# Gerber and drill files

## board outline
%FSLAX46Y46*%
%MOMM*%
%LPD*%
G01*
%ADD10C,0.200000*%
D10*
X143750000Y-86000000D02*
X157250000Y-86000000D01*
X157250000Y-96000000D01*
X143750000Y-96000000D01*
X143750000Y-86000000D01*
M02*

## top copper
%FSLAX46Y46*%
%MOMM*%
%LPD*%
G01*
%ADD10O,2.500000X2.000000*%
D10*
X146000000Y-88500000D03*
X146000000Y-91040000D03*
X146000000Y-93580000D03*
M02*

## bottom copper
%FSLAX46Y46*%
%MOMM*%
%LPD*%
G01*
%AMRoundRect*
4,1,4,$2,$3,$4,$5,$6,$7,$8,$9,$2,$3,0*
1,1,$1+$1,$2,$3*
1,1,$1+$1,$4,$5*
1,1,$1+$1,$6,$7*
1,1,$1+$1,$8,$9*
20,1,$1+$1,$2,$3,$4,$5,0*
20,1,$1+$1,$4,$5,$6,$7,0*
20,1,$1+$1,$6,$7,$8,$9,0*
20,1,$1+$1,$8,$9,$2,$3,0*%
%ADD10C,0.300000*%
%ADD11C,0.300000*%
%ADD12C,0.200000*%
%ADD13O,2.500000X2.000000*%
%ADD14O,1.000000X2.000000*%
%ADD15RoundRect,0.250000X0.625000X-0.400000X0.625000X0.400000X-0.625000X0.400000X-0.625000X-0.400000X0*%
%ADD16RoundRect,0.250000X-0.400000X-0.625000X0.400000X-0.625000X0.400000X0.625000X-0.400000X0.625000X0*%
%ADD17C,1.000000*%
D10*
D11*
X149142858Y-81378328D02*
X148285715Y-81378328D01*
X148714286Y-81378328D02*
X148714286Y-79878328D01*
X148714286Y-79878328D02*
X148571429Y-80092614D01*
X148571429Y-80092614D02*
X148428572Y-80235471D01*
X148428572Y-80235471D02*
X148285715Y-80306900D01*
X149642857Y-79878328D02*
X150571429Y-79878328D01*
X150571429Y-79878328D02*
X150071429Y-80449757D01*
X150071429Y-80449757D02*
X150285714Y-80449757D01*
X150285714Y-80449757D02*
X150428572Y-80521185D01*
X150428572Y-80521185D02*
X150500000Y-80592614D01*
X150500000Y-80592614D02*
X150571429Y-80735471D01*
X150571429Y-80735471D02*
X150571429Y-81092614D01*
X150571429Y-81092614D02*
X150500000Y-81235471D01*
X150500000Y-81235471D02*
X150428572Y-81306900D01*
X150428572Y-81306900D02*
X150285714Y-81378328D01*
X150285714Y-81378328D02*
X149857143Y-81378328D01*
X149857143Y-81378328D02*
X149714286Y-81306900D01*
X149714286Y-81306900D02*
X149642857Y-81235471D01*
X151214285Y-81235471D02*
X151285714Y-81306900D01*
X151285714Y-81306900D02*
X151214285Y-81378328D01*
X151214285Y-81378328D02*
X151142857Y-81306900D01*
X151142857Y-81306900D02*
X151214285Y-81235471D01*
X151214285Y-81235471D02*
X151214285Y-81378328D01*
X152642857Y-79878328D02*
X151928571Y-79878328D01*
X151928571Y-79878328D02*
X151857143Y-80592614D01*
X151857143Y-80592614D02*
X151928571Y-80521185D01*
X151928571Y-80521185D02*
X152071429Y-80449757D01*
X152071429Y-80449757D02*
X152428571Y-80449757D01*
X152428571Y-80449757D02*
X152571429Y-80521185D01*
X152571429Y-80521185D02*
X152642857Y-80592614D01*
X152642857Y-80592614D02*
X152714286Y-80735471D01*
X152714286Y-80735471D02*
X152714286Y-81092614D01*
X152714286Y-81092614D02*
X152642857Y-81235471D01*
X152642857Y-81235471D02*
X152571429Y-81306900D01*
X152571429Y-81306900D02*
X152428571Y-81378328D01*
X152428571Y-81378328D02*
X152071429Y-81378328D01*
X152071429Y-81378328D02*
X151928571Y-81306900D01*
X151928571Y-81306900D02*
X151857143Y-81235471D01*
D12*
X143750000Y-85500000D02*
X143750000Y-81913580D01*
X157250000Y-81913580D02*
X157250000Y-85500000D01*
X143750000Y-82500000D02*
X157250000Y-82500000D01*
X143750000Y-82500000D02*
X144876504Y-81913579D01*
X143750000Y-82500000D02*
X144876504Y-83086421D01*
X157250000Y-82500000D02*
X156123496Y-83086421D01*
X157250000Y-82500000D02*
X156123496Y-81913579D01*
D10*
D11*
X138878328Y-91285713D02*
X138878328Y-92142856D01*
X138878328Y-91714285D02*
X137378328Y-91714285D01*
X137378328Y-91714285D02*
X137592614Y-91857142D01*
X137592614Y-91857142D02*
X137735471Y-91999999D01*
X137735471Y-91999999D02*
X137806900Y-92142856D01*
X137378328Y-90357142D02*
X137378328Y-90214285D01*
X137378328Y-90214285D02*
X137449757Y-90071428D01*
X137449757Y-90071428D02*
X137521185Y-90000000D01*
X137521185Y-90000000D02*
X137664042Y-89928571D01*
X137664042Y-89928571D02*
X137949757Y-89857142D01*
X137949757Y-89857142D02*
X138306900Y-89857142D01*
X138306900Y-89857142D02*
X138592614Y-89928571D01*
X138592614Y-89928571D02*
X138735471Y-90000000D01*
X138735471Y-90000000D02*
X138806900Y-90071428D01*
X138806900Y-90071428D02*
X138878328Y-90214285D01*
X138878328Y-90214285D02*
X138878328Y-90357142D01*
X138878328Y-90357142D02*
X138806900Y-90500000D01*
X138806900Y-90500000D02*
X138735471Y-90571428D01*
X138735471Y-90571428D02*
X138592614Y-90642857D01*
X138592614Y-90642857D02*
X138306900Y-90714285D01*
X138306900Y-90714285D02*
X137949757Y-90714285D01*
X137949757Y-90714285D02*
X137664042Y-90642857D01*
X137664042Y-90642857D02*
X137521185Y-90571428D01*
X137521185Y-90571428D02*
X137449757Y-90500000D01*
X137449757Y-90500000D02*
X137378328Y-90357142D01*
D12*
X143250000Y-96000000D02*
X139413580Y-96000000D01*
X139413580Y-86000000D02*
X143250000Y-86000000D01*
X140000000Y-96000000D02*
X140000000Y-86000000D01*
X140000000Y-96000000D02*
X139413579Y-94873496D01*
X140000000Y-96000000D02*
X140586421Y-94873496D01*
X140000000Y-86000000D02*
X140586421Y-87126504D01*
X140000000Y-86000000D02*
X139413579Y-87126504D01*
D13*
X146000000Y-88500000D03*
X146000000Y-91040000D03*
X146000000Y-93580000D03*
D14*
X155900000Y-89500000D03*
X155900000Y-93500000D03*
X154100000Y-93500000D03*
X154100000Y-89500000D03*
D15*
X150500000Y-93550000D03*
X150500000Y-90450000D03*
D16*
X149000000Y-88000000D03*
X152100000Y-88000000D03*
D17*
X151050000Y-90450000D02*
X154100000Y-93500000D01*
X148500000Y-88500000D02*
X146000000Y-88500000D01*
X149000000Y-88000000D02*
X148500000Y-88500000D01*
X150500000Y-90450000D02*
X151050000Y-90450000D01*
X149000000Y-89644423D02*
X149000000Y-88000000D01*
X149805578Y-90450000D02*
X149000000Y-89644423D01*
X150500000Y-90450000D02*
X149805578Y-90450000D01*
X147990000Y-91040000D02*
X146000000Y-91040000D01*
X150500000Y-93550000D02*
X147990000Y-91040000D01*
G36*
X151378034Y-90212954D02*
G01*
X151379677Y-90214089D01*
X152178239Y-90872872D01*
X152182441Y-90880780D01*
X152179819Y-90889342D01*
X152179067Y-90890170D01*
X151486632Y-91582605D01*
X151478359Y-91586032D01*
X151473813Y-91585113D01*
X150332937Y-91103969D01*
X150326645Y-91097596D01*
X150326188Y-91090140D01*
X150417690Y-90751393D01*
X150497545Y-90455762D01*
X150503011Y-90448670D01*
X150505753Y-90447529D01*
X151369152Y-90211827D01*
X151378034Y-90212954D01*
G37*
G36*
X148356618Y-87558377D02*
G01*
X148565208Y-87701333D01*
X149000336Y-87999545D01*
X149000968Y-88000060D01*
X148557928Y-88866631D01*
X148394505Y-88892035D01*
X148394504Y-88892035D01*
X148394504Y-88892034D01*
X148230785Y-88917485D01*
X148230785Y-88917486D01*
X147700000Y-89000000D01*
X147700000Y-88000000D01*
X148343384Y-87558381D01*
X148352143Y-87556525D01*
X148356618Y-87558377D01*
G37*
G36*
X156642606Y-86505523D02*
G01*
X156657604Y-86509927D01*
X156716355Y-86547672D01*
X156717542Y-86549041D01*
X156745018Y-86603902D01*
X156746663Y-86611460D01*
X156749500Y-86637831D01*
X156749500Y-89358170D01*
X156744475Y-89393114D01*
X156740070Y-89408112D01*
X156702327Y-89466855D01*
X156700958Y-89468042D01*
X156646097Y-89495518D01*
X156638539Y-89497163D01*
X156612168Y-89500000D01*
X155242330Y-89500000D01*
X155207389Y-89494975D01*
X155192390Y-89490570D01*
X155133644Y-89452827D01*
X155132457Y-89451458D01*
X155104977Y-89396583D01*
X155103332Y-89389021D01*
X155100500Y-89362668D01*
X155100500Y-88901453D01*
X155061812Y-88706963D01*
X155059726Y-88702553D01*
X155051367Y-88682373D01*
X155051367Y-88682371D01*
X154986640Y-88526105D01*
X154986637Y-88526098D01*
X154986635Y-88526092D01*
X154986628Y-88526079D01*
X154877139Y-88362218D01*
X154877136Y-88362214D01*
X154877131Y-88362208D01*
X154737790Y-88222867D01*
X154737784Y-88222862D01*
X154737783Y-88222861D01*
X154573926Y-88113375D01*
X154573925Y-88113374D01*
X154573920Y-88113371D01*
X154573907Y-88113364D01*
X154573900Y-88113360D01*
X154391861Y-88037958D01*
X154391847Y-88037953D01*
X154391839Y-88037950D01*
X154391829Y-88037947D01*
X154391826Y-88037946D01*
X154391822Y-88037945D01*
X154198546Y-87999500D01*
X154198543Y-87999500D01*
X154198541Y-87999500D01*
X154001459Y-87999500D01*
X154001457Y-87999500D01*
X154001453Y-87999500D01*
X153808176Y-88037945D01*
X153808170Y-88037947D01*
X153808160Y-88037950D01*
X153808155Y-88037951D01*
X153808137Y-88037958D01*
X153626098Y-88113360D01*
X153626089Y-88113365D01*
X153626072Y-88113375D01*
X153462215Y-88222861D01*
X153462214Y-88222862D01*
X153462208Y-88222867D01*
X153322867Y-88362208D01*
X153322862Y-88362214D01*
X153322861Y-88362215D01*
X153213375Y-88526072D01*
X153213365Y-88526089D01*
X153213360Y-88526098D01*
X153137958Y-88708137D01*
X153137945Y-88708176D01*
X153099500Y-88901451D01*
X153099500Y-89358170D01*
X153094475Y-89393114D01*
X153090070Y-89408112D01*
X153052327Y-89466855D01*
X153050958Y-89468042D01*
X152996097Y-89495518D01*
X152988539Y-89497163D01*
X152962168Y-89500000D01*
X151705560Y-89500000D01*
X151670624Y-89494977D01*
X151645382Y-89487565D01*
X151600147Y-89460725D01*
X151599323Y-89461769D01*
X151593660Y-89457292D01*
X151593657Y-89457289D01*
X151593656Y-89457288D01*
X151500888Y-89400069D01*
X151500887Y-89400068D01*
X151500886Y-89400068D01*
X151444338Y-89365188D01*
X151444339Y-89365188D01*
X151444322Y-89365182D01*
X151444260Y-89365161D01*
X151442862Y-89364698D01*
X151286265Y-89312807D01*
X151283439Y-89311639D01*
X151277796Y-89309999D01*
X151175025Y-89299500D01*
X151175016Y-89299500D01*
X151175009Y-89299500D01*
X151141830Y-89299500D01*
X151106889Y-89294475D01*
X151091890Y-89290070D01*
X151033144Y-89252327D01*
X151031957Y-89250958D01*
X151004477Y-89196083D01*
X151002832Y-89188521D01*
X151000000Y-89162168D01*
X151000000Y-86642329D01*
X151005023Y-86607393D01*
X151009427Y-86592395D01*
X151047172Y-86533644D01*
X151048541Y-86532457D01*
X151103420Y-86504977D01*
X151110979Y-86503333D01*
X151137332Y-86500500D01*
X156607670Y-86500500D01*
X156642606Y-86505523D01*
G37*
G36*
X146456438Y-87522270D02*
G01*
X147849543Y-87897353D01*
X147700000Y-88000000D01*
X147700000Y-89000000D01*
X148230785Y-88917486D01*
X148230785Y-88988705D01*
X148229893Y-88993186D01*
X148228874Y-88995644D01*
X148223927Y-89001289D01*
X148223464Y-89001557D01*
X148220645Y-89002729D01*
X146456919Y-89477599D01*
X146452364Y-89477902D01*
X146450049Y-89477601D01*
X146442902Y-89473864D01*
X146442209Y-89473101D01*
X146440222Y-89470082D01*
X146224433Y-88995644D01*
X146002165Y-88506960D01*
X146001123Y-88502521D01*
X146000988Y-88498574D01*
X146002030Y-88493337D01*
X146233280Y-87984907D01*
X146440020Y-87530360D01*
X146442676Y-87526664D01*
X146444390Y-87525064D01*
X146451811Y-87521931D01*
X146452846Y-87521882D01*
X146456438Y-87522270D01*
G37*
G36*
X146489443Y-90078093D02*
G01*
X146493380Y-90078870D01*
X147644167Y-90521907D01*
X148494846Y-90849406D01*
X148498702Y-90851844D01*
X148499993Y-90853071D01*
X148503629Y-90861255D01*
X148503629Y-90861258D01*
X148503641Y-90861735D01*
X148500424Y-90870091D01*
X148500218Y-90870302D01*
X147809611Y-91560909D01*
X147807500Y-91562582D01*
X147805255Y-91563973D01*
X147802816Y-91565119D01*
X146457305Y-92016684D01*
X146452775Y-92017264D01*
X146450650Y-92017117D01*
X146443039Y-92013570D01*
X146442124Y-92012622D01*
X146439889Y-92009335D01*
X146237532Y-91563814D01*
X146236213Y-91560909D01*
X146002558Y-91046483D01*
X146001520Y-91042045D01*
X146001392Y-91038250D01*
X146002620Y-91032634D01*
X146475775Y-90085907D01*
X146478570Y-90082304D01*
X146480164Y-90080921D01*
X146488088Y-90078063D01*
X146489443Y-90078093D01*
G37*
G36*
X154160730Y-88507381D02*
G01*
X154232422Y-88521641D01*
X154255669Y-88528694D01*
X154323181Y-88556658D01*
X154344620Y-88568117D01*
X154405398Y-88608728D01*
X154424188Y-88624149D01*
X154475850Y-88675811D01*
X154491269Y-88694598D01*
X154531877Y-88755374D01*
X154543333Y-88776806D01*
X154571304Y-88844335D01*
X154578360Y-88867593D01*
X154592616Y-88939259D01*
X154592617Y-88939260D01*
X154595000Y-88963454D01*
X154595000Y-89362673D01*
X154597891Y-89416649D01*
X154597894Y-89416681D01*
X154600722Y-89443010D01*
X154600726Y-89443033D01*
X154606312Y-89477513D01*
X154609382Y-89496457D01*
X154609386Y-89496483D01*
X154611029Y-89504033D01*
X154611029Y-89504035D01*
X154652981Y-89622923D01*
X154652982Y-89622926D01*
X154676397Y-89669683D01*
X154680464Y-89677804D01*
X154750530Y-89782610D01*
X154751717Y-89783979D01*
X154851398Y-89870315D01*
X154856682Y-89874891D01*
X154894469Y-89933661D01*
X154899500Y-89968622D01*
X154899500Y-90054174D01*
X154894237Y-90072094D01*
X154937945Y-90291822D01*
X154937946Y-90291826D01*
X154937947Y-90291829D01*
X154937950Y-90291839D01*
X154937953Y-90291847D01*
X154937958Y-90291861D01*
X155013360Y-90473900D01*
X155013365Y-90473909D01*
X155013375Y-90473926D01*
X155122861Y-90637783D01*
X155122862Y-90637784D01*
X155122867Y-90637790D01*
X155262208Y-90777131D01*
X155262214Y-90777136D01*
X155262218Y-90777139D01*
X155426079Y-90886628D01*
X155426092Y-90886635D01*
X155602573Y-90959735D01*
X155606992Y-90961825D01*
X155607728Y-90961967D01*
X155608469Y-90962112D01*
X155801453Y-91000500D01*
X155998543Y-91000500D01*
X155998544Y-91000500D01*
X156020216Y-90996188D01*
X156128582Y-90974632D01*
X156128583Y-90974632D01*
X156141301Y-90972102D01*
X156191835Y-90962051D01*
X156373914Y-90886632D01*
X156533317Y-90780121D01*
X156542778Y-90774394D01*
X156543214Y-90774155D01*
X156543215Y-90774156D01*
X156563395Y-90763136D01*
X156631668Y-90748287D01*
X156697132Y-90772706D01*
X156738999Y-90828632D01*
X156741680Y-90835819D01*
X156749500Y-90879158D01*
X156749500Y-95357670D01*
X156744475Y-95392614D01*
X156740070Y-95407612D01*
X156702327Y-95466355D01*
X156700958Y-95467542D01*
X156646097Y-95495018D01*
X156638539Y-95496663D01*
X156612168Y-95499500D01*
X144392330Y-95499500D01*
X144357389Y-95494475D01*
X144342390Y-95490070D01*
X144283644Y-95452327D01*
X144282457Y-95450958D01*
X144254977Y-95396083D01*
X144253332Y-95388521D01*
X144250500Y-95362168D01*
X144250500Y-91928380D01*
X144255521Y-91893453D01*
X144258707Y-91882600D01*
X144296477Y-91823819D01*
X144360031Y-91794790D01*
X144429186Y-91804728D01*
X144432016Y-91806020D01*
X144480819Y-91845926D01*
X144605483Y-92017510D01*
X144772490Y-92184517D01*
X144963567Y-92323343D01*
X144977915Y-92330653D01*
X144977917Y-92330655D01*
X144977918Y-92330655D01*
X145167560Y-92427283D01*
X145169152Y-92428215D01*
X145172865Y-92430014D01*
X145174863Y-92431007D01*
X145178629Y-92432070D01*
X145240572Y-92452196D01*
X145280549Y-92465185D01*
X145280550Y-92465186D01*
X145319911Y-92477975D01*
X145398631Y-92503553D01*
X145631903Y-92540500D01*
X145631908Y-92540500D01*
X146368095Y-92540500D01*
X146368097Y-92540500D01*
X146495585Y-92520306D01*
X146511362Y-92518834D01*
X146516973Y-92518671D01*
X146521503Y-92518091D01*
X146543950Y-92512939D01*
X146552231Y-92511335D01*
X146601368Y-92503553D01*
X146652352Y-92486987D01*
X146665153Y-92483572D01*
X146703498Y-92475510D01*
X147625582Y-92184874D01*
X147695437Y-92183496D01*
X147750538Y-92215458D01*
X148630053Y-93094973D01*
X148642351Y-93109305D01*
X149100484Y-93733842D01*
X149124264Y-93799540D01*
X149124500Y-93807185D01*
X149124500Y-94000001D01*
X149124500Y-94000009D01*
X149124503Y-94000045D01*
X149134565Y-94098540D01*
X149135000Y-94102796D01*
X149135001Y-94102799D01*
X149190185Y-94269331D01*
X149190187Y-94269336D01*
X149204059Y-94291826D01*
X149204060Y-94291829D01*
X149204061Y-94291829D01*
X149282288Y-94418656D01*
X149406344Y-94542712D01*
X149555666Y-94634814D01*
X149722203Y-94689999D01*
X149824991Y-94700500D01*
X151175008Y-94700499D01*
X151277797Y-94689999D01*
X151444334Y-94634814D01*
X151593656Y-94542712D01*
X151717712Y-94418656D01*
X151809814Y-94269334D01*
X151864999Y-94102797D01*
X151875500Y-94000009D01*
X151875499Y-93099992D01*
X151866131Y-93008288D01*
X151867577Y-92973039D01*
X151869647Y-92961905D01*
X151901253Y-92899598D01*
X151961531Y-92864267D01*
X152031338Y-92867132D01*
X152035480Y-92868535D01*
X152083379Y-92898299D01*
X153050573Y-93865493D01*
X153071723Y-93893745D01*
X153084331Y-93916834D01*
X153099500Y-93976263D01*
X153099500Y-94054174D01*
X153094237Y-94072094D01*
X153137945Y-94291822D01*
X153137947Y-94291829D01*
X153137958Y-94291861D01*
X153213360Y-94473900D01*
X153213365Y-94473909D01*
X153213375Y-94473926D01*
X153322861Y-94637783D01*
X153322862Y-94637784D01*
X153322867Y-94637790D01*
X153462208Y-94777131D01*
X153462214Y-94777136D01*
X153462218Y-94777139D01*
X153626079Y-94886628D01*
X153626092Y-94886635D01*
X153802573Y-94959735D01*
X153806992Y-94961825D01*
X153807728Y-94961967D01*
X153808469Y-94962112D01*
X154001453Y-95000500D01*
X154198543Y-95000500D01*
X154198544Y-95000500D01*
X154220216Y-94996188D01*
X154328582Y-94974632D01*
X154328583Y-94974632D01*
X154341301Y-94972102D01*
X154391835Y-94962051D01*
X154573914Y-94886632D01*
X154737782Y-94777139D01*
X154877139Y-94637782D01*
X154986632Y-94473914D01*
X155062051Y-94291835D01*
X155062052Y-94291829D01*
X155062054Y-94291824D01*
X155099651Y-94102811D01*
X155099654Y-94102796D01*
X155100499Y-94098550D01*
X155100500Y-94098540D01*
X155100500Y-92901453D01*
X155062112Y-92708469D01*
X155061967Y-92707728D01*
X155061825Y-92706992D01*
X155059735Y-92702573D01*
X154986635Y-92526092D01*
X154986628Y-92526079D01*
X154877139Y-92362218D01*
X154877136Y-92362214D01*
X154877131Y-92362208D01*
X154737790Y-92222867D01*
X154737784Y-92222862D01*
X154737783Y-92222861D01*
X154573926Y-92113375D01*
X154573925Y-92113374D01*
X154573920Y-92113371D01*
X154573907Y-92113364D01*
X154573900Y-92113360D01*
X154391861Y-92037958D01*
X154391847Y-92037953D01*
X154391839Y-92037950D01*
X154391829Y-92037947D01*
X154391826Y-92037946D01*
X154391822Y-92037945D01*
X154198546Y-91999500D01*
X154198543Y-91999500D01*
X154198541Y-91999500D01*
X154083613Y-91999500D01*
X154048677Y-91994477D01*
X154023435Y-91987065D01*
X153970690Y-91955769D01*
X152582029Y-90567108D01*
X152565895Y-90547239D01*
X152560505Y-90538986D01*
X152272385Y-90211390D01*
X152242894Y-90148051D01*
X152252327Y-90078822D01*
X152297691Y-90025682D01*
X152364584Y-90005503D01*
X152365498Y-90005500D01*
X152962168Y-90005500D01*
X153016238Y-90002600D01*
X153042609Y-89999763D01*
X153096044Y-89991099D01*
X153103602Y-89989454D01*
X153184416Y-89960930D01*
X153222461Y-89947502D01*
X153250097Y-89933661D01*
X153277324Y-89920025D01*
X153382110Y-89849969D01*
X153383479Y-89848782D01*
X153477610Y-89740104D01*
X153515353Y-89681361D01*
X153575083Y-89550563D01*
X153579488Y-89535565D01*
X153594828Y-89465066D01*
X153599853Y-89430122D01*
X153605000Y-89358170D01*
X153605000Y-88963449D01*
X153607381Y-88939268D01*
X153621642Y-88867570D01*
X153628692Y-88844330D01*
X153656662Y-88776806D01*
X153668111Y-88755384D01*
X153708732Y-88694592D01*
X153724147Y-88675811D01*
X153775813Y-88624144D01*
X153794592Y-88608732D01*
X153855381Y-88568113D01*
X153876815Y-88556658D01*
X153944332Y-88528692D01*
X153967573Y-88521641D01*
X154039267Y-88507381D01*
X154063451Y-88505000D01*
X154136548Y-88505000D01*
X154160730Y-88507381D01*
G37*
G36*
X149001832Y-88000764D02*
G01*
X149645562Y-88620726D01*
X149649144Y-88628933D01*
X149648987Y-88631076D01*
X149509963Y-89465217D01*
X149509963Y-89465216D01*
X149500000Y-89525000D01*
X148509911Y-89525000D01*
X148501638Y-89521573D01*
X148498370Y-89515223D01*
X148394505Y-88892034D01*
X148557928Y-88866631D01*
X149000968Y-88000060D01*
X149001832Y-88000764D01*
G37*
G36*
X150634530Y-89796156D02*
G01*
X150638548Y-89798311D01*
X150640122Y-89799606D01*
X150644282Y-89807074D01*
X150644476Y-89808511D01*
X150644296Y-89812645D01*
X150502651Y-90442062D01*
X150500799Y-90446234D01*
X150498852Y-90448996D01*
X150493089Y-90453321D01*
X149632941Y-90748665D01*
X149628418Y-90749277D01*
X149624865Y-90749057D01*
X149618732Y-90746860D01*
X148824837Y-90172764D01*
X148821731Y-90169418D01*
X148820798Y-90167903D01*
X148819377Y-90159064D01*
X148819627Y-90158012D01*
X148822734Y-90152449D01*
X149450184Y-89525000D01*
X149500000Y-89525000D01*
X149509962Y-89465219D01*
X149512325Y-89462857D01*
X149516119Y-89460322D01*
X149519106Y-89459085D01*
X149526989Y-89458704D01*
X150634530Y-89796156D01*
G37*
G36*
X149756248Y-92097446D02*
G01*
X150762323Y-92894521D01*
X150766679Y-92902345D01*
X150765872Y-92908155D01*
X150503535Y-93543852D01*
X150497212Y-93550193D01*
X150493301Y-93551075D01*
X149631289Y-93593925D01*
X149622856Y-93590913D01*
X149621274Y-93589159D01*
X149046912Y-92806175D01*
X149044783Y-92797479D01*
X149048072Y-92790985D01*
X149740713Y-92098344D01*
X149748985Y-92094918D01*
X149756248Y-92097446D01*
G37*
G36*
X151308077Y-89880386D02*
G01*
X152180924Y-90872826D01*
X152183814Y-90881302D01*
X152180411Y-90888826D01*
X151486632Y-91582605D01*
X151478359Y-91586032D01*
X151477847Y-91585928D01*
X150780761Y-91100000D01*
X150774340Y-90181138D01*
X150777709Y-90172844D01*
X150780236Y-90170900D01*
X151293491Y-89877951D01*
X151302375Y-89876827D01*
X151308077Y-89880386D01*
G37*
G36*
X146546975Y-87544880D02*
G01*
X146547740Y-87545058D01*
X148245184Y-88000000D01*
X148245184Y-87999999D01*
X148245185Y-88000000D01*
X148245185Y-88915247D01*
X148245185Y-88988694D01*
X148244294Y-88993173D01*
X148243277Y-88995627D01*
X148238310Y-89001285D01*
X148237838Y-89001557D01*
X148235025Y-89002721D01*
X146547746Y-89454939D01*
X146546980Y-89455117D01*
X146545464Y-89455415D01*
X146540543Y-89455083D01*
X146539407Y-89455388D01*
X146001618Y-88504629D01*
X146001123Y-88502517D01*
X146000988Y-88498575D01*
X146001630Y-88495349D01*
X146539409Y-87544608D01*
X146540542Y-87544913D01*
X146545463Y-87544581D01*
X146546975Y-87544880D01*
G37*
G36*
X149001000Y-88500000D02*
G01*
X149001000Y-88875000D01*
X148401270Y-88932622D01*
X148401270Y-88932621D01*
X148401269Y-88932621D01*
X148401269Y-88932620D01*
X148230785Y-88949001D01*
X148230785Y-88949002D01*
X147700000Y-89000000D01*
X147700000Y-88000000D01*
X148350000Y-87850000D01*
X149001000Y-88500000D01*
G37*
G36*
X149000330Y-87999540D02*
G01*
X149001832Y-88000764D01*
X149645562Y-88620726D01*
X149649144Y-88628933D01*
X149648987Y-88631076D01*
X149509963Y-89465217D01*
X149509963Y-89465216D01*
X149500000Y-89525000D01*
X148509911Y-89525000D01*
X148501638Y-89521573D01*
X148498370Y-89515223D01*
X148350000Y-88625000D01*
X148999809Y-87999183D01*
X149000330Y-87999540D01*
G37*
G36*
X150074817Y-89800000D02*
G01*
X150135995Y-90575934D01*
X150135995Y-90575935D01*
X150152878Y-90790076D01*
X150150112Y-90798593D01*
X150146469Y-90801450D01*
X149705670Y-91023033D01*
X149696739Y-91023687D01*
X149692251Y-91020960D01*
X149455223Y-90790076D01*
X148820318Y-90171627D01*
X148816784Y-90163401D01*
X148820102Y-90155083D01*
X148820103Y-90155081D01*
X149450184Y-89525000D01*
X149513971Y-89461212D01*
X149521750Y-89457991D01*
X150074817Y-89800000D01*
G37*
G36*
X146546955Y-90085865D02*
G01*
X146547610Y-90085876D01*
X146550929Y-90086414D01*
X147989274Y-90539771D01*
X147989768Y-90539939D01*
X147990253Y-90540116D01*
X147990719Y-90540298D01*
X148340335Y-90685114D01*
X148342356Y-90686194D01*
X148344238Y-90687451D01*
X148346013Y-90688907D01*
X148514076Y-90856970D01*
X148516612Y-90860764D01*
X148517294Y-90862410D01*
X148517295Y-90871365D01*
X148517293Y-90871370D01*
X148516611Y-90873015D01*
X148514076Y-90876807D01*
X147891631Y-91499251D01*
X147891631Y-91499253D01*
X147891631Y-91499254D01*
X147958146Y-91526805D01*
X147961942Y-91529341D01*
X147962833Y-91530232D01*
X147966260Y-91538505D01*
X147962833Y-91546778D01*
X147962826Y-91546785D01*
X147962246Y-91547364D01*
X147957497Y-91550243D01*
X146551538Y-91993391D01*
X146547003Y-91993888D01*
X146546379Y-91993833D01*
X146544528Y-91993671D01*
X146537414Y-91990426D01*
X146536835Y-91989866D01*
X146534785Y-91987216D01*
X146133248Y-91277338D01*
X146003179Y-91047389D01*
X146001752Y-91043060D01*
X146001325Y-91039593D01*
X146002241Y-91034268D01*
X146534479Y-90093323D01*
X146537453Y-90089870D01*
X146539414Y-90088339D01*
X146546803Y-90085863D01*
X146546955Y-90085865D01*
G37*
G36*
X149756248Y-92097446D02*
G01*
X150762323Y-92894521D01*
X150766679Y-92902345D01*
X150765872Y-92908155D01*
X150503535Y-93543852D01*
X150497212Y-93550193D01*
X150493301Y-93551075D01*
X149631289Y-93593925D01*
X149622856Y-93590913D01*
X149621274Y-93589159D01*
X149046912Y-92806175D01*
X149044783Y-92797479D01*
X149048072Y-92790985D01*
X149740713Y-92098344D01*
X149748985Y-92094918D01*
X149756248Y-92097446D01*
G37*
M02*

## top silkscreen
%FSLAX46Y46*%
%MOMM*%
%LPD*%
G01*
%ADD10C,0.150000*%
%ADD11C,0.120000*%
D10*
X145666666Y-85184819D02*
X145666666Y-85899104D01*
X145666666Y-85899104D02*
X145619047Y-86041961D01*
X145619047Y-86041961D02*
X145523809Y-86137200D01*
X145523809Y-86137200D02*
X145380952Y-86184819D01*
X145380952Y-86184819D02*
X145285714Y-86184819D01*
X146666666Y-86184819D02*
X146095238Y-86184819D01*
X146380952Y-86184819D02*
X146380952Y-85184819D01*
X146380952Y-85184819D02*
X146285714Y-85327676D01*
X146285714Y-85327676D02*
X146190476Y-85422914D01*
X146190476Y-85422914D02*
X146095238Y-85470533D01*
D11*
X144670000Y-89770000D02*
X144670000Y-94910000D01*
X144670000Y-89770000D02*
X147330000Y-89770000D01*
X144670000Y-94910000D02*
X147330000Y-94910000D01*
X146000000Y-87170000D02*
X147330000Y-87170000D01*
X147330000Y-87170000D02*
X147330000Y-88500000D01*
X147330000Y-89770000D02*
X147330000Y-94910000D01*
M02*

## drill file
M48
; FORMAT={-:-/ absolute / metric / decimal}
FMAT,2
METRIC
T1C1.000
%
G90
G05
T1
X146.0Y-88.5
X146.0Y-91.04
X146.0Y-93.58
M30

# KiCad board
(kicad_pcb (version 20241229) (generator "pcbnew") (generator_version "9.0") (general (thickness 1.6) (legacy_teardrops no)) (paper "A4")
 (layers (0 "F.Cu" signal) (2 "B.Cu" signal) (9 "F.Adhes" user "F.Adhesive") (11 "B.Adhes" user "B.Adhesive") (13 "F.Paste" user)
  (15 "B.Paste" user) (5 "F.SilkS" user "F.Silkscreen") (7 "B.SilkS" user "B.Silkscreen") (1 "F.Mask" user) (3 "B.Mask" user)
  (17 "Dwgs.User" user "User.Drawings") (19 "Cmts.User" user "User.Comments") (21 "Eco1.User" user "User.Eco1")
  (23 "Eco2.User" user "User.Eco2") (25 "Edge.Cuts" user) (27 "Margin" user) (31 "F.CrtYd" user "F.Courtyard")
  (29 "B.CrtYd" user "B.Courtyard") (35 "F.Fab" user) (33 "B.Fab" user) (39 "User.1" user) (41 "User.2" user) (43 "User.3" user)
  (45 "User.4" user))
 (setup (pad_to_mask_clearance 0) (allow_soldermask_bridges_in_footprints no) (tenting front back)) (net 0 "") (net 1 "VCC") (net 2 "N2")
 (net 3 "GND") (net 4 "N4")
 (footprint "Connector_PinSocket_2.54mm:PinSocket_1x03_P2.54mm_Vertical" (layer "F.Cu") (at 146 88.5)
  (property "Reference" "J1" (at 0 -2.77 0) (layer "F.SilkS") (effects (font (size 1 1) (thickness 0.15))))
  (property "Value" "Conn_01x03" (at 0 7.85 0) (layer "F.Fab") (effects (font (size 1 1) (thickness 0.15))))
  (fp_line (start -1.33 1.27) (end -1.33 6.41) (stroke (width 0.12) (type solid)) (layer "F.SilkS"))
  (fp_line (start -1.33 1.27) (end 1.33 1.27) (stroke (width 0.12) (type solid)) (layer "F.SilkS"))
  (fp_line (start -1.33 6.41) (end 1.33 6.41) (stroke (width 0.12) (type solid)) (layer "F.SilkS"))
  (fp_line (start 0 -1.33) (end 1.33 -1.33) (stroke (width 0.12) (type solid)) (layer "F.SilkS"))
  (fp_line (start 1.33 -1.33) (end 1.33 0) (stroke (width 0.12) (type solid)) (layer "F.SilkS"))
  (fp_line (start 1.33 1.27) (end 1.33 6.41) (stroke (width 0.12) (type solid)) (layer "F.SilkS"))
  (pad "1" thru_hole oval (at 0 0) (size 2.5 2) (drill 1) (layers "*.Cu" "*.Mask") (remove_unused_layers no) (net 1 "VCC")
   (teardrops (best_length_ratio 0.5) (max_length 1) (best_width_ratio 1) (max_width 2) (curved_edges no) (filter_ratio 0.9) (enabled yes)
    (allow_two_segments yes) (prefer_zone_connections yes)))
  (pad "2" thru_hole oval (at 0 2.54) (size 2.5 2) (drill 1) (layers "*.Cu" "*.Mask") (remove_unused_layers no) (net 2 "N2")
   (teardrops (best_length_ratio 0.5) (max_length 1) (best_width_ratio 1) (max_width 2) (curved_edges no) (filter_ratio 0.9) (enabled yes)
    (allow_two_segments yes) (prefer_zone_connections yes)))
  (pad "3" thru_hole oval (at 0 5.08) (size 2.5 2) (drill 1) (layers "*.Cu" "*.Mask") (remove_unused_layers no) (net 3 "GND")
   (teardrops (best_length_ratio 0.5) (max_length 1) (best_width_ratio 1) (max_width 2) (curved_edges no) (filter_ratio 0.9) (enabled yes)
    (allow_two_segments yes) (prefer_zone_connections yes))))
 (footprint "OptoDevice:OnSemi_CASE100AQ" (layer "B.Cu") (at 155.9 89.5 180)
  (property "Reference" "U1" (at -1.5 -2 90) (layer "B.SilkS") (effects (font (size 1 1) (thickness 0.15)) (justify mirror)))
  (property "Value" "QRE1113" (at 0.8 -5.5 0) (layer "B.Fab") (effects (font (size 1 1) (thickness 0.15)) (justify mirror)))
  (pad "1" smd oval (at 0 0 180) (size 1 2) (layers "B.Cu" "B.Mask" "B.Paste") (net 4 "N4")
   (teardrops (best_length_ratio 0.5) (max_length 1) (best_width_ratio 1) (max_width 2) (curved_edges no) (filter_ratio 0.9) (enabled yes)
    (allow_two_segments yes) (prefer_zone_connections yes)))
  (pad "2" smd oval (at 0 -4 180) (size 1 2) (layers "B.Cu" "B.Mask" "B.Paste") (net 3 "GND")
   (teardrops (best_length_ratio 0.5) (max_length 1) (best_width_ratio 1) (max_width 2) (curved_edges no) (filter_ratio 0.9) (enabled yes)
    (allow_two_segments yes) (prefer_zone_connections yes)))
  (pad "3" smd oval (at 1.8 -4 180) (size 1 2) (layers "B.Cu" "B.Mask" "B.Paste") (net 1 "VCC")
   (teardrops (best_length_ratio 0.5) (max_length 1) (best_width_ratio 1) (max_width 2) (curved_edges no) (filter_ratio 0.9) (enabled yes)
    (allow_two_segments yes) (prefer_zone_connections yes)))
  (pad "4" smd oval (at 1.8 0 180) (size 1 2) (layers "B.Cu" "B.Mask" "B.Paste") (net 3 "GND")
   (teardrops (best_length_ratio 0.5) (max_length 1) (best_width_ratio 1) (max_width 2) (curved_edges no) (filter_ratio 0.9) (enabled yes)
    (allow_two_segments yes) (prefer_zone_connections yes))))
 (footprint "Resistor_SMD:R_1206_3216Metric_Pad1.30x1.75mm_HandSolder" (layer "B.Cu") (at 150.5 92 90)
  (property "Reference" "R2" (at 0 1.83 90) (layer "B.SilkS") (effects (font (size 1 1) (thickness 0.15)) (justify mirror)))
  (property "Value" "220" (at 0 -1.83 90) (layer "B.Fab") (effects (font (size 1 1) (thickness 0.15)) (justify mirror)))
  (pad "1" smd roundrect (at -1.55 0 90) (size 1.3 1.75) (layers "B.Cu" "B.Mask" "B.Paste") (roundrect_rratio 0.192308) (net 2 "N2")
   (teardrops (best_length_ratio 0.5) (max_length 1) (best_width_ratio 1) (max_width 2) (curved_edges no) (filter_ratio 0.9) (enabled yes)
    (allow_two_segments yes) (prefer_zone_connections yes)))
  (pad "2" smd roundrect (at 1.55 0 90) (size 1.3 1.75) (layers "B.Cu" "B.Mask" "B.Paste") (roundrect_rratio 0.192308) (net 1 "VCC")
   (teardrops (best_length_ratio 0.5) (max_length 1) (best_width_ratio 1) (max_width 2) (curved_edges no) (filter_ratio 0.9) (enabled yes)
    (allow_two_segments yes) (prefer_zone_connections yes))))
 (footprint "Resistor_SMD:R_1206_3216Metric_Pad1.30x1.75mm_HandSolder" (layer "B.Cu") (at 150.55 88)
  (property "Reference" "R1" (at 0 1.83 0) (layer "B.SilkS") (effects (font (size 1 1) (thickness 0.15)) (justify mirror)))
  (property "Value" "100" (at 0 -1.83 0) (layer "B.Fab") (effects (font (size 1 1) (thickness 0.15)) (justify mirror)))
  (pad "1" smd roundrect (at -1.55 0) (size 1.3 1.75) (layers "B.Cu" "B.Mask" "B.Paste") (roundrect_rratio 0.192308) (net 1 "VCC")
   (teardrops (best_length_ratio 0.5) (max_length 1) (best_width_ratio 1) (max_width 2) (curved_edges no) (filter_ratio 0.9) (enabled yes)
    (allow_two_segments yes) (prefer_zone_connections yes)))
  (pad "2" smd roundrect (at 1.55 0) (size 1.3 1.75) (layers "B.Cu" "B.Mask" "B.Paste") (roundrect_rratio 0.192308) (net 4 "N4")
   (teardrops (best_length_ratio 0.5) (max_length 1) (best_width_ratio 1) (max_width 2) (curved_edges no) (filter_ratio 0.9) (enabled yes)
    (allow_two_segments yes) (prefer_zone_connections yes))))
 (gr_rect (start 143.75 86) (end 157.25 96) (stroke (width 0.2) (type solid)) (fill no) (layer "Edge.Cuts"))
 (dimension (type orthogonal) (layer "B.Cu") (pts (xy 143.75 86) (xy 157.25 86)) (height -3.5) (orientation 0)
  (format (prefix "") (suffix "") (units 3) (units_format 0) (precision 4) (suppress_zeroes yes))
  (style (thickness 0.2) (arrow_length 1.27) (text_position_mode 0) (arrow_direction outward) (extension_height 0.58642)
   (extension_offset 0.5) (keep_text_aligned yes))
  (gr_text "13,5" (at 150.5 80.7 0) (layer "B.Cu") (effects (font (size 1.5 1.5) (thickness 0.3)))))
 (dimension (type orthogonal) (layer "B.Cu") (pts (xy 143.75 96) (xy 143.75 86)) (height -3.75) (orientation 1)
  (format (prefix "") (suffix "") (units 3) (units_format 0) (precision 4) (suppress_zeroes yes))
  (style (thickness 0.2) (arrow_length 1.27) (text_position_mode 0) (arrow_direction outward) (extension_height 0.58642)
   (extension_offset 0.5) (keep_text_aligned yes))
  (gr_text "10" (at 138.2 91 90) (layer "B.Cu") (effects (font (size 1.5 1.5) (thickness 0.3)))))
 (segment (start 151.05 90.45) (end 154.1 93.5) (width 1) (layer "B.Cu") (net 1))
 (segment (start 148.5 88.5) (end 146 88.5) (width 1) (layer "B.Cu") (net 1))
 (segment (start 149 88) (end 148.5 88.5) (width 1) (layer "B.Cu") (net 1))
 (segment (start 150.5 90.45) (end 151.05 90.45) (width 1) (layer "B.Cu") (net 1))
 (segment (start 149 89.644423) (end 149 88) (width 1) (layer "B.Cu") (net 1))
 (segment (start 149.805578 90.45) (end 149 89.644423) (width 1) (layer "B.Cu") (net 1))
 (segment (start 150.5 90.45) (end 149.805578 90.45) (width 1) (layer "B.Cu") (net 1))
 (segment (start 147.99 91.04) (end 146 91.04) (width 1) (layer "B.Cu") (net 2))
 (segment (start 150.5 93.55) (end 147.99 91.04) (width 1) (layer "B.Cu") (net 2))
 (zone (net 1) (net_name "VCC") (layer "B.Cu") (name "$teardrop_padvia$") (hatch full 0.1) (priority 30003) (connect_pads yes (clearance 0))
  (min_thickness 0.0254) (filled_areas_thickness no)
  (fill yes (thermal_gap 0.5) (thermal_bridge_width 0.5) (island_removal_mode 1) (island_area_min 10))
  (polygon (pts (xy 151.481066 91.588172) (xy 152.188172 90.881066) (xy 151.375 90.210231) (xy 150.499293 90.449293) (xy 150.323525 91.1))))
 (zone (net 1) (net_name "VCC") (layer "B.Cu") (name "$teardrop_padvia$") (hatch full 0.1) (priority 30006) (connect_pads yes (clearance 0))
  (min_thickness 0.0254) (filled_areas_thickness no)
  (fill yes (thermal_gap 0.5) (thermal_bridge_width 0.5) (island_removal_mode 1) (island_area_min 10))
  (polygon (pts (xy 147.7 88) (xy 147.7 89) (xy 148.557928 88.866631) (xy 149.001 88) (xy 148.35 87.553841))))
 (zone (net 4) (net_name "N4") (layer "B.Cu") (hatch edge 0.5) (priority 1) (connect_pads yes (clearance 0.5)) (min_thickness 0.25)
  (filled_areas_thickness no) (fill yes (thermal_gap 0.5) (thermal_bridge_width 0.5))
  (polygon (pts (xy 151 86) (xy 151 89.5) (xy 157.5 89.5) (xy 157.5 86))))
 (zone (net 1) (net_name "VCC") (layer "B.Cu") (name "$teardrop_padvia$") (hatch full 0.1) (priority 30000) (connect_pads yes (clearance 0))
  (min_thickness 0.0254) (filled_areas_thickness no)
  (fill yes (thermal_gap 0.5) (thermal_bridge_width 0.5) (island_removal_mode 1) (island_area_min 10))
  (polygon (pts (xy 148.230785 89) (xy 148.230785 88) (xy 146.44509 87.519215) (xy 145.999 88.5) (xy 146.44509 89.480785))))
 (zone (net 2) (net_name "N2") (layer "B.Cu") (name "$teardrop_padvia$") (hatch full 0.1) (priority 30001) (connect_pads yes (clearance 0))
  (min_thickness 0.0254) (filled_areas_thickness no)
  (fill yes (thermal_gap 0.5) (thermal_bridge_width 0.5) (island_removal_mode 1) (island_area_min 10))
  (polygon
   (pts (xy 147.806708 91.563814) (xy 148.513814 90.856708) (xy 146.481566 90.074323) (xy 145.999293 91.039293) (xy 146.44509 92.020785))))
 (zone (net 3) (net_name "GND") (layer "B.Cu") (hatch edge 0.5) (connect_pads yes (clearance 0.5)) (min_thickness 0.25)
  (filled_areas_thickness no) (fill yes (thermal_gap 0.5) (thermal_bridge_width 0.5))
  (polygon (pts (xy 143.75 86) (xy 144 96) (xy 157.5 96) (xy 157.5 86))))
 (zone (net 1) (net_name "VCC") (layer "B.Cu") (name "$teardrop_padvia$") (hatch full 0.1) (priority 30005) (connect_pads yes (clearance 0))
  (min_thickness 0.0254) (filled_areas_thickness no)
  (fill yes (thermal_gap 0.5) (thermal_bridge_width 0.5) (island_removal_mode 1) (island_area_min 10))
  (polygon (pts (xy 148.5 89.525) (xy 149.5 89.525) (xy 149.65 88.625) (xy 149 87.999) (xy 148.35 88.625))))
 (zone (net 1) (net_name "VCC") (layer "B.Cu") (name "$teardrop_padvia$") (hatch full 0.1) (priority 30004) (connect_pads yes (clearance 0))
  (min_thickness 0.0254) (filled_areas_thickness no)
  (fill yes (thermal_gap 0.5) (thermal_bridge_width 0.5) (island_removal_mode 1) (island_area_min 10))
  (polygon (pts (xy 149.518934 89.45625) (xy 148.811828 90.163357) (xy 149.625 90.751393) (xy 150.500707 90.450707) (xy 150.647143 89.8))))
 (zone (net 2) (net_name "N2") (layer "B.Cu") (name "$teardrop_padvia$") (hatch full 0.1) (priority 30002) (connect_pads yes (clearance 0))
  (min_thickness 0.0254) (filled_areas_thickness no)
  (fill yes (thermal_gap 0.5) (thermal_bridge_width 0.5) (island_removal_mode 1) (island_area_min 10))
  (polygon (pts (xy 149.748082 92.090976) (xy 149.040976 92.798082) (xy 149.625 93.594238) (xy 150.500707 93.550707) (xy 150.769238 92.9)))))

